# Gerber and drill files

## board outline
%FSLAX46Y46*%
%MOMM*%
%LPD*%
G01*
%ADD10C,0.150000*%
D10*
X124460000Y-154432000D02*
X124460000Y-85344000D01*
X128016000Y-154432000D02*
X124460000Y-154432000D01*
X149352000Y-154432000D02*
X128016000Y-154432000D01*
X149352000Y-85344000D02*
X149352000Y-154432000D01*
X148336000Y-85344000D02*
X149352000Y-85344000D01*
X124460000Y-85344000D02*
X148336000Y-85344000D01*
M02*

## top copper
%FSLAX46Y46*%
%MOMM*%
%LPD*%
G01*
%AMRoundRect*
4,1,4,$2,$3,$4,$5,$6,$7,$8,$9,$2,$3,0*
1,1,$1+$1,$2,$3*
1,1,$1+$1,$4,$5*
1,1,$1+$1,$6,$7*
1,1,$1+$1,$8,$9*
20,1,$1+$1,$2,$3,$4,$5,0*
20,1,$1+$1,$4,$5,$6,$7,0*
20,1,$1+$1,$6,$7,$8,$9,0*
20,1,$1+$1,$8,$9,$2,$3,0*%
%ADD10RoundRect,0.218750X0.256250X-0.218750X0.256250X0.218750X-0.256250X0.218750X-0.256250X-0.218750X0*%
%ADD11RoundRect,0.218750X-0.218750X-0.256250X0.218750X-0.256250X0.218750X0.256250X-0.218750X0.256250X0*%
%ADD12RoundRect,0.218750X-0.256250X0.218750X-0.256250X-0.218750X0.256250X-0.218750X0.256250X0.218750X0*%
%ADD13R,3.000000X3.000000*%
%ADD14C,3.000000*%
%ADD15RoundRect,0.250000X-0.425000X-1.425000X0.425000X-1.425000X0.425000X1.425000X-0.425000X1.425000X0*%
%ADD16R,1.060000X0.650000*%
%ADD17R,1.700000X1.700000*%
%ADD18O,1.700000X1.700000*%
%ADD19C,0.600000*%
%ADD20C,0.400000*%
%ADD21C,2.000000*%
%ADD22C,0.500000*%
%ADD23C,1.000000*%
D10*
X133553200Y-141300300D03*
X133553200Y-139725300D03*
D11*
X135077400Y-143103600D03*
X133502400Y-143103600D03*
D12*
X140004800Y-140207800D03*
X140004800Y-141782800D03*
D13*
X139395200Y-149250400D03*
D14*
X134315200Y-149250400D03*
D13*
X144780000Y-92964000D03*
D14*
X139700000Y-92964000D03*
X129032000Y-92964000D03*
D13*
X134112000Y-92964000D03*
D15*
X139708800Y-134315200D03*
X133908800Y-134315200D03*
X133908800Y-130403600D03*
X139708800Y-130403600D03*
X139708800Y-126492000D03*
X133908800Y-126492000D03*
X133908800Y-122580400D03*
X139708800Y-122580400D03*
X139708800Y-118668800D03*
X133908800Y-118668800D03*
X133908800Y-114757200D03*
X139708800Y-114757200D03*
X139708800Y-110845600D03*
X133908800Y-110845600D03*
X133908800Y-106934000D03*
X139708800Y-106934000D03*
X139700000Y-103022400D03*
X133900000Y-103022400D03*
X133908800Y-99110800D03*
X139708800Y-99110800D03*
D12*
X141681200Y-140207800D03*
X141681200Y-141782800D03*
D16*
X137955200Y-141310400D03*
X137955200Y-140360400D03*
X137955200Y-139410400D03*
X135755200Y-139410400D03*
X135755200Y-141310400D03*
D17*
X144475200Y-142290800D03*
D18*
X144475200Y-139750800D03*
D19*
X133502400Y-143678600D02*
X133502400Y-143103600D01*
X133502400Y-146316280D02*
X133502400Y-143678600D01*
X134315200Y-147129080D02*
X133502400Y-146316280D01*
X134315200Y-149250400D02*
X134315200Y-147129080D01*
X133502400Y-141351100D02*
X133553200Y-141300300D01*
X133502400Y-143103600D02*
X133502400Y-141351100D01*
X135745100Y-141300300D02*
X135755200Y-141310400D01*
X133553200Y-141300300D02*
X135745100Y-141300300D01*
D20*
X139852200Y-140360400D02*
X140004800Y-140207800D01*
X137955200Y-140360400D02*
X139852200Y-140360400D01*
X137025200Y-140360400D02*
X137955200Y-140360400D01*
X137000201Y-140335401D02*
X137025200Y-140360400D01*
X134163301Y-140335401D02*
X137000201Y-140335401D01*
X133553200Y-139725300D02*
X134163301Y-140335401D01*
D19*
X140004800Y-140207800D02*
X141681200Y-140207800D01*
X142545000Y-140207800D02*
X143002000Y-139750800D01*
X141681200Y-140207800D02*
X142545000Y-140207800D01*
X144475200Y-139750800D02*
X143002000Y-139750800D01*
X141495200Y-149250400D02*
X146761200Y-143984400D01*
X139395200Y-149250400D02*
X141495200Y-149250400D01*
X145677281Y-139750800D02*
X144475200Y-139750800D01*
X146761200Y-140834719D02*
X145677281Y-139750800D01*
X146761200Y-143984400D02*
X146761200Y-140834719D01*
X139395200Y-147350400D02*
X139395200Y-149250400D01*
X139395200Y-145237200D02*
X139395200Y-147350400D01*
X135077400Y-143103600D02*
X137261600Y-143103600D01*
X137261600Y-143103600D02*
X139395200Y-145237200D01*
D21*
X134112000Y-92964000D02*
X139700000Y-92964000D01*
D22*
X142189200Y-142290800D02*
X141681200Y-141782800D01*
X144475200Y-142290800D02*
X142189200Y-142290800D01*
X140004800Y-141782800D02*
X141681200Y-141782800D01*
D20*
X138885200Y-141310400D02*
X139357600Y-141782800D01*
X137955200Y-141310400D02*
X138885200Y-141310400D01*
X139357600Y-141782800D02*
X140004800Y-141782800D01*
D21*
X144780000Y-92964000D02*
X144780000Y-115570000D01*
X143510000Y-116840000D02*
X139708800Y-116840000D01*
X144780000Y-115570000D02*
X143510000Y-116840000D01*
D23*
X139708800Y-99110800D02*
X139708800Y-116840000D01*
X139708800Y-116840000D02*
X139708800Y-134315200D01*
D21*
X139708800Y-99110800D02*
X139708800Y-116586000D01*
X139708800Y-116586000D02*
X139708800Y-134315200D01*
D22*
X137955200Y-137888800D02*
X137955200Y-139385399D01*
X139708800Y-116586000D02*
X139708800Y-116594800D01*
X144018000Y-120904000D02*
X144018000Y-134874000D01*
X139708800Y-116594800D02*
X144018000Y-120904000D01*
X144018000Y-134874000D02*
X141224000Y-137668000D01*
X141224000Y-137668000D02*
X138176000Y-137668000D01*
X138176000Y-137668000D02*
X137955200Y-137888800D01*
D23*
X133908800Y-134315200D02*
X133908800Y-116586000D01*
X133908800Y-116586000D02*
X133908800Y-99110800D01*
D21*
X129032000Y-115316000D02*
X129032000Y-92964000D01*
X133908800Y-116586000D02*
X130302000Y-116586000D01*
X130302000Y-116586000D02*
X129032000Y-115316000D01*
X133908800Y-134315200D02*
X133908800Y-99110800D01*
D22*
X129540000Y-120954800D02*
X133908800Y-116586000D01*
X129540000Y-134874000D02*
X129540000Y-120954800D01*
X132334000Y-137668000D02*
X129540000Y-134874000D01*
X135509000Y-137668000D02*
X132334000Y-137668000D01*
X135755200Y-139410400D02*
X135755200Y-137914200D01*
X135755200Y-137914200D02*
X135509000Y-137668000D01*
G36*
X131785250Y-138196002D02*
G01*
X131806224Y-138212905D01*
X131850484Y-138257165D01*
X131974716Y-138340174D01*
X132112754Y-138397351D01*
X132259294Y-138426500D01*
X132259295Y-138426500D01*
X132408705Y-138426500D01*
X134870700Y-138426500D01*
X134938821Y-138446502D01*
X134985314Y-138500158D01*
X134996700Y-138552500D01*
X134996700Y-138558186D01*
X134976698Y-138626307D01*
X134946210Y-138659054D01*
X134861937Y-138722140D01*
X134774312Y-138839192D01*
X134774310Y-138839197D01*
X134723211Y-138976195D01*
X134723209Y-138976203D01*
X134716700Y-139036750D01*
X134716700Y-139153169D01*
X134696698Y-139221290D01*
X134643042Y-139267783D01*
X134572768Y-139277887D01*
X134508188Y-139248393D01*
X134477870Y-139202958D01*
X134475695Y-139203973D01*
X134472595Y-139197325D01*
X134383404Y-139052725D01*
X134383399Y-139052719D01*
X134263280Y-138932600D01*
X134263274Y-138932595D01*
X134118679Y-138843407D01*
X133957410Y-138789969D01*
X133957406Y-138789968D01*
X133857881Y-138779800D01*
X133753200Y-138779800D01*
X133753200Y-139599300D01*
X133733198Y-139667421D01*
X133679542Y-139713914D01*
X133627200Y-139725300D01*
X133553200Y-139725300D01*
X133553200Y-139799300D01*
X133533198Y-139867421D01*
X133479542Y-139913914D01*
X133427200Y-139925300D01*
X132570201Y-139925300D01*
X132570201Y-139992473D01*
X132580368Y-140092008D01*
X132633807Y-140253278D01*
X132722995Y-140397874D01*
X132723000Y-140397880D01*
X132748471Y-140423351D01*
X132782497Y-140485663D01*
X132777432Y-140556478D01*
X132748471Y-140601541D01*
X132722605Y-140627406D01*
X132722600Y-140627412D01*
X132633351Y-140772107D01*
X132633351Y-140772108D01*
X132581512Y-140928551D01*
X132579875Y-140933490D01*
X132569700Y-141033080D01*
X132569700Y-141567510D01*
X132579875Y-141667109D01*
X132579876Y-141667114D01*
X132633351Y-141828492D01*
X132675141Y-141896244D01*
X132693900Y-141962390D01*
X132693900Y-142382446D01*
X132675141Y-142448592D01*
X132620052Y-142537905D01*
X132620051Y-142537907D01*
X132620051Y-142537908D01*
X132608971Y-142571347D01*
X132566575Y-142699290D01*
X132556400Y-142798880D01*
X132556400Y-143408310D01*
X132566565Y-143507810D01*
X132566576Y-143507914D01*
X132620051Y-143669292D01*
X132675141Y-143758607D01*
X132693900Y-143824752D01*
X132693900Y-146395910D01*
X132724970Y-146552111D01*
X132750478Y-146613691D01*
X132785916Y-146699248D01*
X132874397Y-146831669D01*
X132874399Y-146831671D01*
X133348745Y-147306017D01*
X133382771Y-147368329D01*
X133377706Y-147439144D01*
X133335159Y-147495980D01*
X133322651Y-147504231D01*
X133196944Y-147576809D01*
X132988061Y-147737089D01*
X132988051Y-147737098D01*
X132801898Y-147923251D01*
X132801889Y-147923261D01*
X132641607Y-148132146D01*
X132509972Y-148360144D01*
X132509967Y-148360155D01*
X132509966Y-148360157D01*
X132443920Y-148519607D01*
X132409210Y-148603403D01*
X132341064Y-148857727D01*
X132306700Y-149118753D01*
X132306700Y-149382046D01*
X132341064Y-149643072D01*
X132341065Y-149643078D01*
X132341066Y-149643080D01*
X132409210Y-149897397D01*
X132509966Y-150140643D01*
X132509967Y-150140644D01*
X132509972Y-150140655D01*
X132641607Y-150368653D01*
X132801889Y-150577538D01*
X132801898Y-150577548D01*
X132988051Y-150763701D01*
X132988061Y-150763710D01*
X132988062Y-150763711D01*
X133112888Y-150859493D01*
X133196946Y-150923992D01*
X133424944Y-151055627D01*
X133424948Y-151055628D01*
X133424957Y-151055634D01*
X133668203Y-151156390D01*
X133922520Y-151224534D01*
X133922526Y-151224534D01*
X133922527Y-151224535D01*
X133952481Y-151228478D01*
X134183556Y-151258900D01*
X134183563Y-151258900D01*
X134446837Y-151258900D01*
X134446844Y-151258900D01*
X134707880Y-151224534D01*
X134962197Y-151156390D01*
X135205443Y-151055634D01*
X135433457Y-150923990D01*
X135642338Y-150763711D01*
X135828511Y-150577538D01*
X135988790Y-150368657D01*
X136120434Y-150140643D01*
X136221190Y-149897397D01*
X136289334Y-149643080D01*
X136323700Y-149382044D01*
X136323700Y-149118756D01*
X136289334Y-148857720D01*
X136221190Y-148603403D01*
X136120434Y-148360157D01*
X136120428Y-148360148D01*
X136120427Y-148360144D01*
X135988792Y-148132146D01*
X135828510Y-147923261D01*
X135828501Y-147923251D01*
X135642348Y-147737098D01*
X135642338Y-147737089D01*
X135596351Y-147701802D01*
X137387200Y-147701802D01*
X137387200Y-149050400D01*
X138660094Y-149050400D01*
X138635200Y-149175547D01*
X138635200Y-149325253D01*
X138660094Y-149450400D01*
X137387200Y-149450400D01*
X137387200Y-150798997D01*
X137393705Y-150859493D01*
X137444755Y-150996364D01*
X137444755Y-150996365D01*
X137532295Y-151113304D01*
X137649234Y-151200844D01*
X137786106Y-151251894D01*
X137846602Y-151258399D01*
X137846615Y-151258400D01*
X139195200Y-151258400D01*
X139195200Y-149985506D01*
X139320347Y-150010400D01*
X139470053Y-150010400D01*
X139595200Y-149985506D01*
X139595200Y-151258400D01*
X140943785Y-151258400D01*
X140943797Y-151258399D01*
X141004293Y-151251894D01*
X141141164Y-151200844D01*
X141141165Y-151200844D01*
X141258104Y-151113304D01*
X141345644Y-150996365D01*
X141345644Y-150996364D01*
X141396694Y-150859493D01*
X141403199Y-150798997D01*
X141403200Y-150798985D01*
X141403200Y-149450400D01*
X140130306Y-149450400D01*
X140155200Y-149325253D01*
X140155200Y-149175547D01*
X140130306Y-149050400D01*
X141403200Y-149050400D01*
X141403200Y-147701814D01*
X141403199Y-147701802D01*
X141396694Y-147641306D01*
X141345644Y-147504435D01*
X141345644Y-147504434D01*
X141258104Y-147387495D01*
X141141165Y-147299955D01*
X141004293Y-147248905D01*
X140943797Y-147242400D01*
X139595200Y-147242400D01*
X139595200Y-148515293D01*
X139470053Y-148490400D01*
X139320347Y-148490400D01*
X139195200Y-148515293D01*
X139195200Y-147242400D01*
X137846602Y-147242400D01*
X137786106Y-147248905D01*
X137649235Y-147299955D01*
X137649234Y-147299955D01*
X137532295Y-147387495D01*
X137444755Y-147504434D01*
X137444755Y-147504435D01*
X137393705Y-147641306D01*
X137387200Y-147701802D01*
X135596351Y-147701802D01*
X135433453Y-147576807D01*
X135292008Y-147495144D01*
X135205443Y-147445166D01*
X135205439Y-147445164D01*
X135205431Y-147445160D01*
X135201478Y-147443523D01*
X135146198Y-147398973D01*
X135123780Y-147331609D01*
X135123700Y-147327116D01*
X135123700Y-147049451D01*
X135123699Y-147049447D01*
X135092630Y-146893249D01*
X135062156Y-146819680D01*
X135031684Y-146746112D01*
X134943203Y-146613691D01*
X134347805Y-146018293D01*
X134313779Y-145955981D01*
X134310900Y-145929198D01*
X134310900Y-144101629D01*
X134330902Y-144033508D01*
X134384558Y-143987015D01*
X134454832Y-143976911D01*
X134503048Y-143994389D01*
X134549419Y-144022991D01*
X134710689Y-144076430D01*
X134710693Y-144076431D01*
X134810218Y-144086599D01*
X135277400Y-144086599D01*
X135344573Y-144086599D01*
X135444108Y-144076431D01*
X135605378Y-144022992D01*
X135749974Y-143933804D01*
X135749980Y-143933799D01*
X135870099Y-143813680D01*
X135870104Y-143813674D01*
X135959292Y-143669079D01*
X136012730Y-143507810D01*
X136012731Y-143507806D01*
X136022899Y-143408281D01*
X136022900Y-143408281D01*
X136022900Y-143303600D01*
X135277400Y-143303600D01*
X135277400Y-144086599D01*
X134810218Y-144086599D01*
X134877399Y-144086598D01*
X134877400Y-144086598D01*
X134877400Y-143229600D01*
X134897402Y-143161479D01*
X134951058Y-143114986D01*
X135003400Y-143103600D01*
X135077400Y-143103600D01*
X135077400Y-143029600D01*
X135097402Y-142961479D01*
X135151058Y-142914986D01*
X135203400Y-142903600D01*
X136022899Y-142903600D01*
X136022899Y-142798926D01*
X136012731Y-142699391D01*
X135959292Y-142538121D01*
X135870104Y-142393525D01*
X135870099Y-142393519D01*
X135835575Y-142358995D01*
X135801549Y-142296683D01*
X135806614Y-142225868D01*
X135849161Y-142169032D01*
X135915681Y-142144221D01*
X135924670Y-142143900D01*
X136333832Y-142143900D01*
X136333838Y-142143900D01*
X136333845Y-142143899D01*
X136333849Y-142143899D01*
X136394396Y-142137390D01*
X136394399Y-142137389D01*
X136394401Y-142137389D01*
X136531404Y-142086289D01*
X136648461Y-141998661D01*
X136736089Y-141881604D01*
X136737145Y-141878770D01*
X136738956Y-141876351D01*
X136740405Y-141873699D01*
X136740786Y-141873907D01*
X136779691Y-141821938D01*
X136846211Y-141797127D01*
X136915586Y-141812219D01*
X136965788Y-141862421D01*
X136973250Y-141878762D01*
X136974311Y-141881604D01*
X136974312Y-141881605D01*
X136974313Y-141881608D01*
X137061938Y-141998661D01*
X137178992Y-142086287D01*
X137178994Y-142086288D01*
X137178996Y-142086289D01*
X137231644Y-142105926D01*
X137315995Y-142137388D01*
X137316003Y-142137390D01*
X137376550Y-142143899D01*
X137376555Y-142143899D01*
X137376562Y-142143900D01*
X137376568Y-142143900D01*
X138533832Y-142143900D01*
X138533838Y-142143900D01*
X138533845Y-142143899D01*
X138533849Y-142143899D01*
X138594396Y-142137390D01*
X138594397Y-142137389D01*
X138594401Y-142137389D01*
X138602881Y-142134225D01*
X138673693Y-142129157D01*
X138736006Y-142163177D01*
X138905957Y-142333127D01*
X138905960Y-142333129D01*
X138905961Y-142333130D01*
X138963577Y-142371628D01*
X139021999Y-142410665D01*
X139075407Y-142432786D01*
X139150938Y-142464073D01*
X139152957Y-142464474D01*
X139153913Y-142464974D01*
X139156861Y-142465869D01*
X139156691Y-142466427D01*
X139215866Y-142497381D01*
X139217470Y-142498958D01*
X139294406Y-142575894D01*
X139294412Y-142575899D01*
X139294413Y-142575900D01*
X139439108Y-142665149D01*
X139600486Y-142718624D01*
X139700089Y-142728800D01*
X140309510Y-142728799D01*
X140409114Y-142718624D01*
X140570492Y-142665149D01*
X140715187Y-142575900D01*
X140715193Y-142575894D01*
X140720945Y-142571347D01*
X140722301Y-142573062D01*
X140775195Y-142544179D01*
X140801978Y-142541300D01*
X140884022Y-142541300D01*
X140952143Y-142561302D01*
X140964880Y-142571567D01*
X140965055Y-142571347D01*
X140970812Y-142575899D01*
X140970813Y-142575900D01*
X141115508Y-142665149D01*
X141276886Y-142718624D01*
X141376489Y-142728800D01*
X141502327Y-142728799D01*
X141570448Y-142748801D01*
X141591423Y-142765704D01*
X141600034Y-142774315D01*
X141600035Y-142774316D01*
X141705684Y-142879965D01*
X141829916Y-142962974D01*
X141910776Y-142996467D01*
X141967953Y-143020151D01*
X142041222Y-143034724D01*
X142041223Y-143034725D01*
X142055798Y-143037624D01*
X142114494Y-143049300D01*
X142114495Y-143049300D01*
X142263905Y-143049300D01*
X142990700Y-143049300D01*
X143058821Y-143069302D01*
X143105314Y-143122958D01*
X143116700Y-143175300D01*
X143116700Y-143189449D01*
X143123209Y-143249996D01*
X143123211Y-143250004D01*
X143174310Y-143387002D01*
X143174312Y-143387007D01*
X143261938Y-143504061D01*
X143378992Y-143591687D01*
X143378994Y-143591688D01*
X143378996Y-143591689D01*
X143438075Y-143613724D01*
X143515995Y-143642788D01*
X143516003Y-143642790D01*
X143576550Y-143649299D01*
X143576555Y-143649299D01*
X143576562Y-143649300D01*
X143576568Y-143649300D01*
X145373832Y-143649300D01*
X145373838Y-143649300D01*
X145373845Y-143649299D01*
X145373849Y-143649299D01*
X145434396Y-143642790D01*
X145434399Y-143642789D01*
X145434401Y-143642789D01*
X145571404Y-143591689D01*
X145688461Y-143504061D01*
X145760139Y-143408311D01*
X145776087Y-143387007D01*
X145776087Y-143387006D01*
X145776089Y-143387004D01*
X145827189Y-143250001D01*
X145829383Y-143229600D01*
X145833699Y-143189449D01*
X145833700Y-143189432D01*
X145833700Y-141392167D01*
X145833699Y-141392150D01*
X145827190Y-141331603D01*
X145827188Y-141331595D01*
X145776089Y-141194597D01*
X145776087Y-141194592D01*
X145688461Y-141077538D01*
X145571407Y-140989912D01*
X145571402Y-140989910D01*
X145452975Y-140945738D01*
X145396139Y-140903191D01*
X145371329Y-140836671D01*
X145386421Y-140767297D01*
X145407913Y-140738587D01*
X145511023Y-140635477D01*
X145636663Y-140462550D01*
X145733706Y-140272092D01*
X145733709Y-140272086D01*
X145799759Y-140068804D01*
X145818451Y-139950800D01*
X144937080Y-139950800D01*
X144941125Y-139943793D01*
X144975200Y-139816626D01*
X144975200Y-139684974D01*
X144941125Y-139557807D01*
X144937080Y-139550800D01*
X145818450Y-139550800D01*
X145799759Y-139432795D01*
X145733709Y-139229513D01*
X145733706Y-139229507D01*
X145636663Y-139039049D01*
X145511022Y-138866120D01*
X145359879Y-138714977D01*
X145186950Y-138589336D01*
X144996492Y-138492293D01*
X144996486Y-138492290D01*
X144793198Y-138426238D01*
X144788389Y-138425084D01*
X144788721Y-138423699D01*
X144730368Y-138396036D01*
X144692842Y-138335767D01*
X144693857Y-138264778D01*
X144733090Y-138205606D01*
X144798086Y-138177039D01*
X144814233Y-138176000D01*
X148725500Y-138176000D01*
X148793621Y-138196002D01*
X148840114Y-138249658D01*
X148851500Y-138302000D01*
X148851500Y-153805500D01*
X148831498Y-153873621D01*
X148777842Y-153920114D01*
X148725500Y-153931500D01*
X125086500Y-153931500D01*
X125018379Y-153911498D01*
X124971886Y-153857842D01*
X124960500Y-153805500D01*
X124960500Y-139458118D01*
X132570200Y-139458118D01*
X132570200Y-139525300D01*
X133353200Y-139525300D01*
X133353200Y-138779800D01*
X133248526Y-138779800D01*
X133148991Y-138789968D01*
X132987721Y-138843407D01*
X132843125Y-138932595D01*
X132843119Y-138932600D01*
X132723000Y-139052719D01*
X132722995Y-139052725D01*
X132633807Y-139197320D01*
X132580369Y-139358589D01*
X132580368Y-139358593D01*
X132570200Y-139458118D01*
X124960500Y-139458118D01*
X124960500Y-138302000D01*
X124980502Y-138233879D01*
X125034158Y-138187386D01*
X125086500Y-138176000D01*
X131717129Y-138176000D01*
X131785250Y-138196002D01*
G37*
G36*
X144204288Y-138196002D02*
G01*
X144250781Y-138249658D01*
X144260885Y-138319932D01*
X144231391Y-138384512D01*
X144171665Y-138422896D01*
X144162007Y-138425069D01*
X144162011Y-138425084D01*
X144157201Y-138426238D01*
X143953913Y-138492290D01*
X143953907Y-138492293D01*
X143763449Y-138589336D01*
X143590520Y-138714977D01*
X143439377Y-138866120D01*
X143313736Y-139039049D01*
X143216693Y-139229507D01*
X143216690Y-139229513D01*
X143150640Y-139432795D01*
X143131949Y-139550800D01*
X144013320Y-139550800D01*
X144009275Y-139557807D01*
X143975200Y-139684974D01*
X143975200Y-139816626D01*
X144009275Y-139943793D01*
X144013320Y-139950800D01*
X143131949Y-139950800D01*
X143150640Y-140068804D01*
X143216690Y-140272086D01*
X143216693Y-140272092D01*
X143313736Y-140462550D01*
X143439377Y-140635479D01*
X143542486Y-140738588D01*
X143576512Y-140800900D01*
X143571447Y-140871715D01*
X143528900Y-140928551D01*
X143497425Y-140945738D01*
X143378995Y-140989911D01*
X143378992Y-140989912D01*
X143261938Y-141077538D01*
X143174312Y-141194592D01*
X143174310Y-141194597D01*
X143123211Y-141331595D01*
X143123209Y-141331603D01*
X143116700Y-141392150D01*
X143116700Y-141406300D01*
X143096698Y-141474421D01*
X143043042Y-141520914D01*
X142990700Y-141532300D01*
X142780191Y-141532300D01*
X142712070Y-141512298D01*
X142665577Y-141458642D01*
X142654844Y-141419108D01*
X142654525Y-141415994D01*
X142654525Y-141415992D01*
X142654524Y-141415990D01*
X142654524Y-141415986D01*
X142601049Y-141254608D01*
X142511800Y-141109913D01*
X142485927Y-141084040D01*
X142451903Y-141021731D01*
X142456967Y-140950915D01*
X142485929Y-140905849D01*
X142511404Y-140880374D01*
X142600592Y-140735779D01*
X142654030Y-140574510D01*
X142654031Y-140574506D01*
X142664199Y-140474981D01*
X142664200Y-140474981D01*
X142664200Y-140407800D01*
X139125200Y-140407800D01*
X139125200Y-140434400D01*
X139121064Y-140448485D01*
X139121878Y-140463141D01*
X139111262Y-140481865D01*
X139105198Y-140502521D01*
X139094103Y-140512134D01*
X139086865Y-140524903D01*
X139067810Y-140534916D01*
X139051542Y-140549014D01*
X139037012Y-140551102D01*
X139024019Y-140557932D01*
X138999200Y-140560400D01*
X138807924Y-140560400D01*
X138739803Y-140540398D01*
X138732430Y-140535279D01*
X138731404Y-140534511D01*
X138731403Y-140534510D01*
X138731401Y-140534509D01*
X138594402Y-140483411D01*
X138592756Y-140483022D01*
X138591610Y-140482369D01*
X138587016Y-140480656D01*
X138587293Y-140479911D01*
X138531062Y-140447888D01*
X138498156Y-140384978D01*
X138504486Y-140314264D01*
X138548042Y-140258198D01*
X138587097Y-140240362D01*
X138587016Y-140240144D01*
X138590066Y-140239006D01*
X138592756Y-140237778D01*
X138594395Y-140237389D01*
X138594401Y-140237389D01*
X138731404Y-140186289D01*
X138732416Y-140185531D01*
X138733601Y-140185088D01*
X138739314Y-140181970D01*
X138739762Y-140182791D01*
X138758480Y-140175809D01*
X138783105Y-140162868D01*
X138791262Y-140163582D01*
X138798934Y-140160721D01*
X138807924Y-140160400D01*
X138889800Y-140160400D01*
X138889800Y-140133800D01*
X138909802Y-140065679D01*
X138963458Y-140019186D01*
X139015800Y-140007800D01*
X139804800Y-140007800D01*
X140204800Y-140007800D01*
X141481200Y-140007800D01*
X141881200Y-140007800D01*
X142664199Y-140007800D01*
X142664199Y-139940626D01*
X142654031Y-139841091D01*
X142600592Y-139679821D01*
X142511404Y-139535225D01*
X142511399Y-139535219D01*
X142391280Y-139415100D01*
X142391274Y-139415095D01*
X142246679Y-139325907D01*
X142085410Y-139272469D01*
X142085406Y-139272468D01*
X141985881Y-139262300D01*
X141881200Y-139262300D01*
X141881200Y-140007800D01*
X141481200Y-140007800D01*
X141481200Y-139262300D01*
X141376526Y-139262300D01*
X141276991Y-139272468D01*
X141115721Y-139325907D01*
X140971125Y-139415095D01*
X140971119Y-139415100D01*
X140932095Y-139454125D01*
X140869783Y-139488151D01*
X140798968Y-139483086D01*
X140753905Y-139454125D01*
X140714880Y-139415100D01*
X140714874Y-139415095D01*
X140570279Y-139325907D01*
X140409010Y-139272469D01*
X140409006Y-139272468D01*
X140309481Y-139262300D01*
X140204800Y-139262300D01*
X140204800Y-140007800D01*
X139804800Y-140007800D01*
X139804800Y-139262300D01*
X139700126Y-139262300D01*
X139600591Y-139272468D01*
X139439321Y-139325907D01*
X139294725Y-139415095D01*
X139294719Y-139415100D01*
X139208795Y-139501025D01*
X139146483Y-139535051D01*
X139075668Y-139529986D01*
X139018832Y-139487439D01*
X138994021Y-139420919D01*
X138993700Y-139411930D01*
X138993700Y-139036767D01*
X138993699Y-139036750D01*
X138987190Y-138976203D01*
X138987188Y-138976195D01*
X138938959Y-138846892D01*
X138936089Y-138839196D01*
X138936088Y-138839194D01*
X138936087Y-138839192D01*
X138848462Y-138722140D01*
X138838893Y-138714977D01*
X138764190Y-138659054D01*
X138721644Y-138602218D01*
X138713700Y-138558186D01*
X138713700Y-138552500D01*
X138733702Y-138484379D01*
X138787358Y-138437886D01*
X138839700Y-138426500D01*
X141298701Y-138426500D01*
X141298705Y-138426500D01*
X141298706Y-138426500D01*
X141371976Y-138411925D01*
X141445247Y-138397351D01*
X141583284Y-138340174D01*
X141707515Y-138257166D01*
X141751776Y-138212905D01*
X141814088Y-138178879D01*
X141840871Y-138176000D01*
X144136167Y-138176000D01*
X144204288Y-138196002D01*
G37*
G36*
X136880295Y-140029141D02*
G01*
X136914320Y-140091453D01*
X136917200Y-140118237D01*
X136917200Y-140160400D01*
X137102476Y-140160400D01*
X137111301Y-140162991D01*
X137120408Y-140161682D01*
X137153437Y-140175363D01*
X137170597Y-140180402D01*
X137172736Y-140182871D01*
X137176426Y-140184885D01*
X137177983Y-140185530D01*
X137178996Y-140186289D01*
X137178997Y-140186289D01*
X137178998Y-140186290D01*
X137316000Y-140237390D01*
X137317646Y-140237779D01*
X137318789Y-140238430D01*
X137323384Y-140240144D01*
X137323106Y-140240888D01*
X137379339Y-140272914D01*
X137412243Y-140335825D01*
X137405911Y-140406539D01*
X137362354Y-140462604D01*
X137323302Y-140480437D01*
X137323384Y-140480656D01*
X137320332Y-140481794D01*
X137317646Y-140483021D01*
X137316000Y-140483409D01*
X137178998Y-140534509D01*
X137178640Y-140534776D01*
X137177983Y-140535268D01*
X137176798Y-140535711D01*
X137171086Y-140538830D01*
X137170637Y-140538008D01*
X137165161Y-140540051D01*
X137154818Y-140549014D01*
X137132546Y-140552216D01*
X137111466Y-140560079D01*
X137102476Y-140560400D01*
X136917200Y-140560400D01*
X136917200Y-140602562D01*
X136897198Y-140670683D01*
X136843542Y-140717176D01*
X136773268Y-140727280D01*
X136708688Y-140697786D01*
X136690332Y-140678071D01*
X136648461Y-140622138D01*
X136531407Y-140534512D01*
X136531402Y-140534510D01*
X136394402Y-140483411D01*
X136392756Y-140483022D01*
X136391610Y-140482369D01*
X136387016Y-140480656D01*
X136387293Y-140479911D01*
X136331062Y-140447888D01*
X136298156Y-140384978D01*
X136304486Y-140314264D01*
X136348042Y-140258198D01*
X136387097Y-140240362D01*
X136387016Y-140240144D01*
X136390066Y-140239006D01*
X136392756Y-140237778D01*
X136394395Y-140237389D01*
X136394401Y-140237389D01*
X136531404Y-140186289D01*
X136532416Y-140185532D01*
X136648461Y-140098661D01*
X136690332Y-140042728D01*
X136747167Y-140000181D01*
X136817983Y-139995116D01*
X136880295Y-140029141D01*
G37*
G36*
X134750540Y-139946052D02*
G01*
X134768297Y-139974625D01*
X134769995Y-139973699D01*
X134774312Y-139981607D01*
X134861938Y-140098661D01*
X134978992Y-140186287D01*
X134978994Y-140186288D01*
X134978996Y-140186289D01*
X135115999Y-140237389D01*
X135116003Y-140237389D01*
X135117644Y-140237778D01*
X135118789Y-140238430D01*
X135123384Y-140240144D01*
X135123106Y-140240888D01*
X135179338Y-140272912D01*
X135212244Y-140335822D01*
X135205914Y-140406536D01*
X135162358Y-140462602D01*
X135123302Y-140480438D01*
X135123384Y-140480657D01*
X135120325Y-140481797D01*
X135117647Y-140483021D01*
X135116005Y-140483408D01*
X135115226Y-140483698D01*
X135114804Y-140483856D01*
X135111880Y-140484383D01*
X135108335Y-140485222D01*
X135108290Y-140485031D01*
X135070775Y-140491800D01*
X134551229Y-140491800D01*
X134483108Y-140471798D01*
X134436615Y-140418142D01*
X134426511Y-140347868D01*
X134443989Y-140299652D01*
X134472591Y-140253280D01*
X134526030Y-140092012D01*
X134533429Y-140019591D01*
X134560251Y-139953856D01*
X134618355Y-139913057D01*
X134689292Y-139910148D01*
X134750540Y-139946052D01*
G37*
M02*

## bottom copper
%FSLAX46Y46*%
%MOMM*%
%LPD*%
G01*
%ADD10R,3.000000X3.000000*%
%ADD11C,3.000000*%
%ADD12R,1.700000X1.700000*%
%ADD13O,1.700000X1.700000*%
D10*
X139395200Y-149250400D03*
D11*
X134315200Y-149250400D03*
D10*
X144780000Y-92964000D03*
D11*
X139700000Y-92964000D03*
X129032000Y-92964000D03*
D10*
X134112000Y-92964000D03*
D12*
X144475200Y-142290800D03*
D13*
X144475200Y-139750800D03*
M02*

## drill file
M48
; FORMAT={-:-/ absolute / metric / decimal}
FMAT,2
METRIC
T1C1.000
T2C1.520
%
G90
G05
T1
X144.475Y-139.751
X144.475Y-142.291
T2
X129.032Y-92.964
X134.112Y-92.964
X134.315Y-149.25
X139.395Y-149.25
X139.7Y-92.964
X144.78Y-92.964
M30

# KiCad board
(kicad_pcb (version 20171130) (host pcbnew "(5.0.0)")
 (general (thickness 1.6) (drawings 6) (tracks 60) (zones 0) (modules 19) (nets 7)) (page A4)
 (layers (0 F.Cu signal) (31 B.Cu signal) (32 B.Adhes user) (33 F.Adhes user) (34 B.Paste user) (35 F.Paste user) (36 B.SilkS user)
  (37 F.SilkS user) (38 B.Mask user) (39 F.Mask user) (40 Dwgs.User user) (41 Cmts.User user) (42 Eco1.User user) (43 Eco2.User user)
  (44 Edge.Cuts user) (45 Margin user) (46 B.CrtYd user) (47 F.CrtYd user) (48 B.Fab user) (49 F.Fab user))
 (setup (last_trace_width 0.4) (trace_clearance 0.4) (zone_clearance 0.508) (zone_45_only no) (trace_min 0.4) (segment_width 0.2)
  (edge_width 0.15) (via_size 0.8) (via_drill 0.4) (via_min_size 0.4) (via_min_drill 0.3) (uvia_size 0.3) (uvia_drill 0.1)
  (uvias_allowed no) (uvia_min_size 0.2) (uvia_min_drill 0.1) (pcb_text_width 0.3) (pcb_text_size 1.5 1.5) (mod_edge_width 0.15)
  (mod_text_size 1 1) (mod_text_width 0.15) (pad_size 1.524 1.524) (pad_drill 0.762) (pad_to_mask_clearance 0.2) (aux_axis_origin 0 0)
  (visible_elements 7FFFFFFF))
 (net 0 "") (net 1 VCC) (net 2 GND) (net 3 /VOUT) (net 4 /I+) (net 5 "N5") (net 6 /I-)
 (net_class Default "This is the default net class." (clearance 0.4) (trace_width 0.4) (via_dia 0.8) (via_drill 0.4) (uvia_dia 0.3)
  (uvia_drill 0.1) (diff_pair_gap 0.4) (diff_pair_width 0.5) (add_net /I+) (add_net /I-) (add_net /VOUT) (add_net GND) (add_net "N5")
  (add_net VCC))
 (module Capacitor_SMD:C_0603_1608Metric (layer F.Cu) (at 133.5532 140.5128 90)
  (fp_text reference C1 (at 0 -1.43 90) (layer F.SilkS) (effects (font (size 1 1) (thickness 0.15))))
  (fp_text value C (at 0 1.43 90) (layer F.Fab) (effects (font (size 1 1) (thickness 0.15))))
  (pad 1 smd roundrect (at -0.7875 0 90) (size 0.875 0.95) (layers F.Cu F.Paste F.Mask) (roundrect_rratio 0.25) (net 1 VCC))
  (pad 2 smd roundrect (at 0.7875 0 90) (size 0.875 0.95) (layers F.Cu F.Paste F.Mask) (roundrect_rratio 0.25) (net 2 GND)))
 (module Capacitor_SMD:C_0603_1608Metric (layer F.Cu) (at 134.2899 143.1036)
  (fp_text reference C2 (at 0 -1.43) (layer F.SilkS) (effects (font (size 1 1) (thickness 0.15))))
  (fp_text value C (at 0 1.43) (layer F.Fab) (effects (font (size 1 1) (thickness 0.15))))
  (pad 2 smd roundrect (at 0.7875 0) (size 0.875 0.95) (layers F.Cu F.Paste F.Mask) (roundrect_rratio 0.25) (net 2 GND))
  (pad 1 smd roundrect (at -0.7875 0) (size 0.875 0.95) (layers F.Cu F.Paste F.Mask) (roundrect_rratio 0.25) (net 1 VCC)))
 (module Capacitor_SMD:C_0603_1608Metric (layer F.Cu) (at 140.0048 140.9953 270)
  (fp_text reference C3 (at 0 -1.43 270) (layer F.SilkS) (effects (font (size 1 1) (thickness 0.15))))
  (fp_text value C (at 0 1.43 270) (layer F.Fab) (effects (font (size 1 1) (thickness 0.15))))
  (pad 1 smd roundrect (at -0.7875 0 270) (size 0.875 0.95) (layers F.Cu F.Paste F.Mask) (roundrect_rratio 0.25) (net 2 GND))
  (pad 2 smd roundrect (at 0.7875 0 270) (size 0.875 0.95) (layers F.Cu F.Paste F.Mask) (roundrect_rratio 0.25) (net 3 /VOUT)))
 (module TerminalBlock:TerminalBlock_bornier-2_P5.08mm (layer F.Cu) (at 139.3952 149.2504 180)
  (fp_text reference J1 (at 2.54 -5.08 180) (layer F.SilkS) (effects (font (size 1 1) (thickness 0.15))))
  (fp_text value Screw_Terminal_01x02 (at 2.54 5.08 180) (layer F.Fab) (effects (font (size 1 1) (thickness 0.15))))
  (pad 1 thru_hole rect (at 0 0 180) (size 3 3) (drill 1.52) (layers *.Cu *.Mask) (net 2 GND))
  (pad 2 thru_hole circle (at 5.08 0 180) (size 3 3) (drill 1.52) (layers *.Cu *.Mask) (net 1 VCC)))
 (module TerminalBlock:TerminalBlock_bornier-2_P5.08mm (layer F.Cu) (at 144.78 92.964 180)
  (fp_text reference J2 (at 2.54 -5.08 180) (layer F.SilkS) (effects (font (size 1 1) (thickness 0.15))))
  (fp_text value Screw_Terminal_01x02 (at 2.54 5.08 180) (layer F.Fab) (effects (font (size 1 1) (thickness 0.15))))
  (pad 1 thru_hole rect (at 0 0 180) (size 3 3) (drill 1.52) (layers *.Cu *.Mask) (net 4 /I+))
  (pad 2 thru_hole circle (at 5.08 0 180) (size 3 3) (drill 1.52) (layers *.Cu *.Mask) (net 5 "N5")))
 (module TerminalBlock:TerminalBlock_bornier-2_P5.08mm (layer F.Cu) (at 134.112 92.964 180)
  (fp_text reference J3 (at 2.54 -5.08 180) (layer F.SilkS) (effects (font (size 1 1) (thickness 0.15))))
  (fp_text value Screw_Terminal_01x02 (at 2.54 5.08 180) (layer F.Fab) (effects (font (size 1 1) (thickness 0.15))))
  (pad 2 thru_hole circle (at 5.08 0 180) (size 3 3) (drill 1.52) (layers *.Cu *.Mask) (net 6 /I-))
  (pad 1 thru_hole rect (at 0 0 180) (size 3 3) (drill 1.52) (layers *.Cu *.Mask) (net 5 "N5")))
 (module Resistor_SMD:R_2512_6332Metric (layer F.Cu) (at 136.8088 134.3152)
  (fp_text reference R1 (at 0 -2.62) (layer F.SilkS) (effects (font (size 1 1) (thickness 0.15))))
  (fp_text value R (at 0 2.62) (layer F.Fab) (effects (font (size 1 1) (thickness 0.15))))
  (pad 2 smd roundrect (at 2.9 0) (size 1.35 3.35) (layers F.Cu F.Paste F.Mask) (roundrect_rratio 0.185185) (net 4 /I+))
  (pad 1 smd roundrect (at -2.9 0) (size 1.35 3.35) (layers F.Cu F.Paste F.Mask) (roundrect_rratio 0.185185) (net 6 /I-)))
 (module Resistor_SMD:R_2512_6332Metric (layer F.Cu) (at 136.8088 130.4036)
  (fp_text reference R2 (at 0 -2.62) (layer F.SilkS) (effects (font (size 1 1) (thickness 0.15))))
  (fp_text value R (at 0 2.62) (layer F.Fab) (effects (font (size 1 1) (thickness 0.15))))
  (pad 1 smd roundrect (at -2.9 0) (size 1.35 3.35) (layers F.Cu F.Paste F.Mask) (roundrect_rratio 0.185185) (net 6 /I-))
  (pad 2 smd roundrect (at 2.9 0) (size 1.35 3.35) (layers F.Cu F.Paste F.Mask) (roundrect_rratio 0.185185) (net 4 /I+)))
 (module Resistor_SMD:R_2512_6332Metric (layer F.Cu) (at 136.8088 126.492)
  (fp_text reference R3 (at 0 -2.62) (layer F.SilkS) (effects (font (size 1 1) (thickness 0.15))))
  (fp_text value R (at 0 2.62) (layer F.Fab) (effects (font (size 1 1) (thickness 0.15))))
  (pad 2 smd roundrect (at 2.9 0) (size 1.35 3.35) (layers F.Cu F.Paste F.Mask) (roundrect_rratio 0.185185) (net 4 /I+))
  (pad 1 smd roundrect (at -2.9 0) (size 1.35 3.35) (layers F.Cu F.Paste F.Mask) (roundrect_rratio 0.185185) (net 6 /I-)))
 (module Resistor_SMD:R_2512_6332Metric (layer F.Cu) (at 136.8088 122.5804)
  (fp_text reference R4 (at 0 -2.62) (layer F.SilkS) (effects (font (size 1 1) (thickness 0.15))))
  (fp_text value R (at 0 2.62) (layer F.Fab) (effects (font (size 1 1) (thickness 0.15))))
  (pad 1 smd roundrect (at -2.9 0) (size 1.35 3.35) (layers F.Cu F.Paste F.Mask) (roundrect_rratio 0.185185) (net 6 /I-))
  (pad 2 smd roundrect (at 2.9 0) (size 1.35 3.35) (layers F.Cu F.Paste F.Mask) (roundrect_rratio 0.185185) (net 4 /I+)))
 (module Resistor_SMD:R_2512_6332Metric (layer F.Cu) (at 136.8088 118.6688)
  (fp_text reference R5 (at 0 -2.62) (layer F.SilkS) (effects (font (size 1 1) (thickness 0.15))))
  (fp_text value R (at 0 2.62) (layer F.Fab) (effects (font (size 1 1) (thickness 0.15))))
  (pad 2 smd roundrect (at 2.9 0) (size 1.35 3.35) (layers F.Cu F.Paste F.Mask) (roundrect_rratio 0.185185) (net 4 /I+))
  (pad 1 smd roundrect (at -2.9 0) (size 1.35 3.35) (layers F.Cu F.Paste F.Mask) (roundrect_rratio 0.185185) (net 6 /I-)))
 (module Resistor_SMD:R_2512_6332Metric (layer F.Cu) (at 136.8088 114.7572)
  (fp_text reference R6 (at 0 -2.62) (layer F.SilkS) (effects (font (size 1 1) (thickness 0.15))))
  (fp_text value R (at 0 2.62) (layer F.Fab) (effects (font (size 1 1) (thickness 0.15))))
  (pad 1 smd roundrect (at -2.9 0) (size 1.35 3.35) (layers F.Cu F.Paste F.Mask) (roundrect_rratio 0.185185) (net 6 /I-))
  (pad 2 smd roundrect (at 2.9 0) (size 1.35 3.35) (layers F.Cu F.Paste F.Mask) (roundrect_rratio 0.185185) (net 4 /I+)))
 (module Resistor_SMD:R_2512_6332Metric (layer F.Cu) (at 136.8088 110.8456)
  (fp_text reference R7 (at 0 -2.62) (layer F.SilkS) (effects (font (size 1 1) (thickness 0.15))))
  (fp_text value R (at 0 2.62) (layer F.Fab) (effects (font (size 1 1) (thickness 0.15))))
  (pad 2 smd roundrect (at 2.9 0) (size 1.35 3.35) (layers F.Cu F.Paste F.Mask) (roundrect_rratio 0.185185) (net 4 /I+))
  (pad 1 smd roundrect (at -2.9 0) (size 1.35 3.35) (layers F.Cu F.Paste F.Mask) (roundrect_rratio 0.185185) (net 6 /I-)))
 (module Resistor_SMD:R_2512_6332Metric (layer F.Cu) (at 136.8088 106.934)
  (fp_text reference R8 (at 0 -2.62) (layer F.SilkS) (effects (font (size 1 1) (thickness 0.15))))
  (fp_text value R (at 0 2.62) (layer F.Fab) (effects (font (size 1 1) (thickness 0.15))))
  (pad 1 smd roundrect (at -2.9 0) (size 1.35 3.35) (layers F.Cu F.Paste F.Mask) (roundrect_rratio 0.185185) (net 6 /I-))
  (pad 2 smd roundrect (at 2.9 0) (size 1.35 3.35) (layers F.Cu F.Paste F.Mask) (roundrect_rratio 0.185185) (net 4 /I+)))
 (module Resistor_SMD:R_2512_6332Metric (layer F.Cu) (at 136.8 103.0224)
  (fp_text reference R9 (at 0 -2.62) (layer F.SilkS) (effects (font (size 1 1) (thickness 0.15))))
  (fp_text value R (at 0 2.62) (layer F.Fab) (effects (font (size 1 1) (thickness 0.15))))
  (pad 2 smd roundrect (at 2.9 0) (size 1.35 3.35) (layers F.Cu F.Paste F.Mask) (roundrect_rratio 0.185185) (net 4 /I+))
  (pad 1 smd roundrect (at -2.9 0) (size 1.35 3.35) (layers F.Cu F.Paste F.Mask) (roundrect_rratio 0.185185) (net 6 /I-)))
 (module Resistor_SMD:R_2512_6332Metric (layer F.Cu) (at 136.8088 99.1108)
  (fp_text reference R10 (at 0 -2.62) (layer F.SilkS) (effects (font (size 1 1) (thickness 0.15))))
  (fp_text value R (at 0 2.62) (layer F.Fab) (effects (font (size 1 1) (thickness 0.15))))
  (pad 1 smd roundrect (at -2.9 0) (size 1.35 3.35) (layers F.Cu F.Paste F.Mask) (roundrect_rratio 0.185185) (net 6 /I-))
  (pad 2 smd roundrect (at 2.9 0) (size 1.35 3.35) (layers F.Cu F.Paste F.Mask) (roundrect_rratio 0.185185) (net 4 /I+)))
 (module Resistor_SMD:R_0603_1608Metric (layer F.Cu) (at 141.6812 140.9953 270)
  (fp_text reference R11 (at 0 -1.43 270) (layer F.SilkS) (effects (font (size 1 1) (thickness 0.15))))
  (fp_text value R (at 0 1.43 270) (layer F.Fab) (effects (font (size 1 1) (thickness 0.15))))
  (pad 1 smd roundrect (at -0.7875 0 270) (size 0.875 0.95) (layers F.Cu F.Paste F.Mask) (roundrect_rratio 0.25) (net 2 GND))
  (pad 2 smd roundrect (at 0.7875 0 270) (size 0.875 0.95) (layers F.Cu F.Paste F.Mask) (roundrect_rratio 0.25) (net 3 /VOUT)))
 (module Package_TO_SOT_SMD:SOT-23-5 (layer F.Cu) (at 136.8552 140.3604 180)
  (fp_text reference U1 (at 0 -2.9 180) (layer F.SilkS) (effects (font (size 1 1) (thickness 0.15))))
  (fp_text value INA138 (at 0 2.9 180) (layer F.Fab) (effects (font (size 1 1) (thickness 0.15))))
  (pad 1 smd rect (at -1.1 -0.95 180) (size 1.06 0.65) (layers F.Cu F.Paste F.Mask) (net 3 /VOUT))
  (pad 2 smd rect (at -1.1 0 180) (size 1.06 0.65) (layers F.Cu F.Paste F.Mask) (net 2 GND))
  (pad 3 smd rect (at -1.1 0.95 180) (size 1.06 0.65) (layers F.Cu F.Paste F.Mask) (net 4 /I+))
  (pad 4 smd rect (at 1.1 0.95 180) (size 1.06 0.65) (layers F.Cu F.Paste F.Mask) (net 6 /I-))
  (pad 5 smd rect (at 1.1 -0.95 180) (size 1.06 0.65) (layers F.Cu F.Paste F.Mask) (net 1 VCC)))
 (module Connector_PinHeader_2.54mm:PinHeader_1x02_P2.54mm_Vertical (layer F.Cu) (at 144.4752 142.2908 180)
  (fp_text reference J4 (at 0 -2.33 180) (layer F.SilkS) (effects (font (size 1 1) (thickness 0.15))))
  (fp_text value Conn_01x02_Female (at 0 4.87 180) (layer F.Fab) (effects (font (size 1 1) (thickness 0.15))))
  (pad 1 thru_hole rect (at 0 0 180) (size 1.7 1.7) (drill 1) (layers *.Cu *.Mask) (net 3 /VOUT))
  (pad 2 thru_hole oval (at 0 2.54 180) (size 1.7 1.7) (drill 1) (layers *.Cu *.Mask) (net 2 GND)))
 (gr_line (start 124.46 154.432) (end 124.46 85.344) (layer Edge.Cuts) (width 0.15))
 (gr_line (start 128.016 154.432) (end 124.46 154.432) (layer Edge.Cuts) (width 0.15))
 (gr_line (start 149.352 154.432) (end 128.016 154.432) (layer Edge.Cuts) (width 0.15))
 (gr_line (start 149.352 85.344) (end 149.352 154.432) (layer Edge.Cuts) (width 0.15))
 (gr_line (start 148.336 85.344) (end 149.352 85.344) (layer Edge.Cuts) (width 0.15))
 (gr_line (start 124.46 85.344) (end 148.336 85.344) (layer Edge.Cuts) (width 0.15))
 (segment (start 133.5024 143.6786) (end 133.5024 143.1036) (width 0.6) (layer F.Cu) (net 1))
 (segment (start 133.5024 146.31628) (end 133.5024 143.6786) (width 0.6) (layer F.Cu) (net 1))
 (segment (start 134.3152 147.12908) (end 133.5024 146.31628) (width 0.6) (layer F.Cu) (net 1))
 (segment (start 134.3152 149.2504) (end 134.3152 147.12908) (width 0.6) (layer F.Cu) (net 1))
 (segment (start 133.5024 141.3511) (end 133.5532 141.3003) (width 0.6) (layer F.Cu) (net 1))
 (segment (start 133.5024 143.1036) (end 133.5024 141.3511) (width 0.6) (layer F.Cu) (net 1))
 (segment (start 135.7451 141.3003) (end 135.7552 141.3104) (width 0.6) (layer F.Cu) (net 1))
 (segment (start 133.5532 141.3003) (end 135.7451 141.3003) (width 0.6) (layer F.Cu) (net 1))
 (segment (start 139.8522 140.3604) (end 140.0048 140.2078) (width 0.4) (layer F.Cu) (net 2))
 (segment (start 137.9552 140.3604) (end 139.8522 140.3604) (width 0.4) (layer F.Cu) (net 2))
 (segment (start 137.0252 140.3604) (end 137.9552 140.3604) (width 0.4) (layer F.Cu) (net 2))
 (segment (start 137.000201 140.335401) (end 137.0252 140.3604) (width 0.4) (layer F.Cu) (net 2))
 (segment (start 134.163301 140.335401) (end 137.000201 140.335401) (width 0.4) (layer F.Cu) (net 2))
 (segment (start 133.5532 139.7253) (end 134.163301 140.335401) (width 0.4) (layer F.Cu) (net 2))
 (segment (start 140.0048 140.2078) (end 141.6812 140.2078) (width 0.6) (layer F.Cu) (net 2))
 (segment (start 142.545 140.2078) (end 143.002 139.7508) (width 0.6) (layer F.Cu) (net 2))
 (segment (start 141.6812 140.2078) (end 142.545 140.2078) (width 0.6) (layer F.Cu) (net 2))
 (segment (start 144.4752 139.7508) (end 143.002 139.7508) (width 0.6) (layer F.Cu) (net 2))
 (segment (start 141.4952 149.2504) (end 146.7612 143.9844) (width 0.6) (layer F.Cu) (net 2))
 (segment (start 139.3952 149.2504) (end 141.4952 149.2504) (width 0.6) (layer F.Cu) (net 2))
 (segment (start 145.677281 139.7508) (end 144.4752 139.7508) (width 0.6) (layer F.Cu) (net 2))
 (segment (start 146.7612 140.834719) (end 145.677281 139.7508) (width 0.6) (layer F.Cu) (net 2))
 (segment (start 146.7612 143.9844) (end 146.7612 140.834719) (width 0.6) (layer F.Cu) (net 2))
 (segment (start 139.3952 147.3504) (end 139.3952 149.2504) (width 0.6) (layer F.Cu) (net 2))
 (segment (start 139.3952 145.2372) (end 139.3952 147.3504) (width 0.6) (layer F.Cu) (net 2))
 (segment (start 135.0774 143.1036) (end 137.2616 143.1036) (width 0.6) (layer F.Cu) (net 2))
 (segment (start 137.2616 143.1036) (end 139.3952 145.2372) (width 0.6) (layer F.Cu) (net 2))
 (segment (start 134.112 92.964) (end 139.7 92.964) (width 2) (layer F.Cu) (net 5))
 (segment (start 142.1892 142.2908) (end 141.6812 141.7828) (width 0.5) (layer F.Cu) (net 3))
 (segment (start 144.4752 142.2908) (end 142.1892 142.2908) (width 0.5) (layer F.Cu) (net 3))
 (segment (start 140.0048 141.7828) (end 141.6812 141.7828) (width 0.5) (layer F.Cu) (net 3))
 (segment (start 138.8852 141.3104) (end 139.3576 141.7828) (width 0.4) (layer F.Cu) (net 3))
 (segment (start 137.9552 141.3104) (end 138.8852 141.3104) (width 0.4) (layer F.Cu) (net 3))
 (segment (start 139.3576 141.7828) (end 140.0048 141.7828) (width 0.4) (layer F.Cu) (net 3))
 (segment (start 144.78 92.964) (end 144.78 115.57) (width 2) (layer F.Cu) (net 4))
 (segment (start 143.51 116.84) (end 139.7088 116.84) (width 2) (layer F.Cu) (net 4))
 (segment (start 144.78 115.57) (end 143.51 116.84) (width 2) (layer F.Cu) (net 4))
 (segment (start 139.7088 99.1108) (end 139.7088 116.84) (width 1) (layer F.Cu) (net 4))
 (segment (start 139.7088 116.84) (end 139.7088 134.3152) (width 1) (layer F.Cu) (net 4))
 (segment (start 139.7088 99.1108) (end 139.7088 116.586) (width 2) (layer F.Cu) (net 4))
 (segment (start 139.7088 116.586) (end 139.7088 134.3152) (width 2) (layer F.Cu) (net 4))
 (segment (start 137.9552 137.8888) (end 137.9552 139.385399) (width 0.5) (layer F.Cu) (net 4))
 (segment (start 139.7088 116.586) (end 139.7088 116.5948) (width 0.5) (layer F.Cu) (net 4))
 (segment (start 144.018 120.904) (end 144.018 134.874) (width 0.5) (layer F.Cu) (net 4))
 (segment (start 139.7088 116.5948) (end 144.018 120.904) (width 0.5) (layer F.Cu) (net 4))
 (segment (start 144.018 134.874) (end 141.224 137.668) (width 0.5) (layer F.Cu) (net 4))
 (segment (start 141.224 137.668) (end 138.176 137.668) (width 0.5) (layer F.Cu) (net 4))
 (segment (start 138.176 137.668) (end 137.9552 137.8888) (width 0.5) (layer F.Cu) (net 4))
 (segment (start 133.9088 134.3152) (end 133.9088 116.586) (width 1) (layer F.Cu) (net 6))
 (segment (start 133.9088 116.586) (end 133.9088 99.1108) (width 1) (layer F.Cu) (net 6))
 (segment (start 129.032 115.316) (end 129.032 92.964) (width 2) (layer F.Cu) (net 6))
 (segment (start 133.9088 116.586) (end 130.302 116.586) (width 2) (layer F.Cu) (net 6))
 (segment (start 130.302 116.586) (end 129.032 115.316) (width 2) (layer F.Cu) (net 6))
 (segment (start 133.9088 134.3152) (end 133.9088 99.1108) (width 2) (layer F.Cu) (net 6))
 (segment (start 129.54 120.9548) (end 133.9088 116.586) (width 0.5) (layer F.Cu) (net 6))
 (segment (start 129.54 134.874) (end 129.54 120.9548) (width 0.5) (layer F.Cu) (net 6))
 (segment (start 132.334 137.668) (end 129.54 134.874) (width 0.5) (layer F.Cu) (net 6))
 (segment (start 135.509 137.668) (end 132.334 137.668) (width 0.5) (layer F.Cu) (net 6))
 (segment (start 135.7552 139.4104) (end 135.7552 137.9142) (width 0.5) (layer F.Cu) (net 6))
 (segment (start 135.7552 137.9142) (end 135.509 137.668) (width 0.5) (layer F.Cu) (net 6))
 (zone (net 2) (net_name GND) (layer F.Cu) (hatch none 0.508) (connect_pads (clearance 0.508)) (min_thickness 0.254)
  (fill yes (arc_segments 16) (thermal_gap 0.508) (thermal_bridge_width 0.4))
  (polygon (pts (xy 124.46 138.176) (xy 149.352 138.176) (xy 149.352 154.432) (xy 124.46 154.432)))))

